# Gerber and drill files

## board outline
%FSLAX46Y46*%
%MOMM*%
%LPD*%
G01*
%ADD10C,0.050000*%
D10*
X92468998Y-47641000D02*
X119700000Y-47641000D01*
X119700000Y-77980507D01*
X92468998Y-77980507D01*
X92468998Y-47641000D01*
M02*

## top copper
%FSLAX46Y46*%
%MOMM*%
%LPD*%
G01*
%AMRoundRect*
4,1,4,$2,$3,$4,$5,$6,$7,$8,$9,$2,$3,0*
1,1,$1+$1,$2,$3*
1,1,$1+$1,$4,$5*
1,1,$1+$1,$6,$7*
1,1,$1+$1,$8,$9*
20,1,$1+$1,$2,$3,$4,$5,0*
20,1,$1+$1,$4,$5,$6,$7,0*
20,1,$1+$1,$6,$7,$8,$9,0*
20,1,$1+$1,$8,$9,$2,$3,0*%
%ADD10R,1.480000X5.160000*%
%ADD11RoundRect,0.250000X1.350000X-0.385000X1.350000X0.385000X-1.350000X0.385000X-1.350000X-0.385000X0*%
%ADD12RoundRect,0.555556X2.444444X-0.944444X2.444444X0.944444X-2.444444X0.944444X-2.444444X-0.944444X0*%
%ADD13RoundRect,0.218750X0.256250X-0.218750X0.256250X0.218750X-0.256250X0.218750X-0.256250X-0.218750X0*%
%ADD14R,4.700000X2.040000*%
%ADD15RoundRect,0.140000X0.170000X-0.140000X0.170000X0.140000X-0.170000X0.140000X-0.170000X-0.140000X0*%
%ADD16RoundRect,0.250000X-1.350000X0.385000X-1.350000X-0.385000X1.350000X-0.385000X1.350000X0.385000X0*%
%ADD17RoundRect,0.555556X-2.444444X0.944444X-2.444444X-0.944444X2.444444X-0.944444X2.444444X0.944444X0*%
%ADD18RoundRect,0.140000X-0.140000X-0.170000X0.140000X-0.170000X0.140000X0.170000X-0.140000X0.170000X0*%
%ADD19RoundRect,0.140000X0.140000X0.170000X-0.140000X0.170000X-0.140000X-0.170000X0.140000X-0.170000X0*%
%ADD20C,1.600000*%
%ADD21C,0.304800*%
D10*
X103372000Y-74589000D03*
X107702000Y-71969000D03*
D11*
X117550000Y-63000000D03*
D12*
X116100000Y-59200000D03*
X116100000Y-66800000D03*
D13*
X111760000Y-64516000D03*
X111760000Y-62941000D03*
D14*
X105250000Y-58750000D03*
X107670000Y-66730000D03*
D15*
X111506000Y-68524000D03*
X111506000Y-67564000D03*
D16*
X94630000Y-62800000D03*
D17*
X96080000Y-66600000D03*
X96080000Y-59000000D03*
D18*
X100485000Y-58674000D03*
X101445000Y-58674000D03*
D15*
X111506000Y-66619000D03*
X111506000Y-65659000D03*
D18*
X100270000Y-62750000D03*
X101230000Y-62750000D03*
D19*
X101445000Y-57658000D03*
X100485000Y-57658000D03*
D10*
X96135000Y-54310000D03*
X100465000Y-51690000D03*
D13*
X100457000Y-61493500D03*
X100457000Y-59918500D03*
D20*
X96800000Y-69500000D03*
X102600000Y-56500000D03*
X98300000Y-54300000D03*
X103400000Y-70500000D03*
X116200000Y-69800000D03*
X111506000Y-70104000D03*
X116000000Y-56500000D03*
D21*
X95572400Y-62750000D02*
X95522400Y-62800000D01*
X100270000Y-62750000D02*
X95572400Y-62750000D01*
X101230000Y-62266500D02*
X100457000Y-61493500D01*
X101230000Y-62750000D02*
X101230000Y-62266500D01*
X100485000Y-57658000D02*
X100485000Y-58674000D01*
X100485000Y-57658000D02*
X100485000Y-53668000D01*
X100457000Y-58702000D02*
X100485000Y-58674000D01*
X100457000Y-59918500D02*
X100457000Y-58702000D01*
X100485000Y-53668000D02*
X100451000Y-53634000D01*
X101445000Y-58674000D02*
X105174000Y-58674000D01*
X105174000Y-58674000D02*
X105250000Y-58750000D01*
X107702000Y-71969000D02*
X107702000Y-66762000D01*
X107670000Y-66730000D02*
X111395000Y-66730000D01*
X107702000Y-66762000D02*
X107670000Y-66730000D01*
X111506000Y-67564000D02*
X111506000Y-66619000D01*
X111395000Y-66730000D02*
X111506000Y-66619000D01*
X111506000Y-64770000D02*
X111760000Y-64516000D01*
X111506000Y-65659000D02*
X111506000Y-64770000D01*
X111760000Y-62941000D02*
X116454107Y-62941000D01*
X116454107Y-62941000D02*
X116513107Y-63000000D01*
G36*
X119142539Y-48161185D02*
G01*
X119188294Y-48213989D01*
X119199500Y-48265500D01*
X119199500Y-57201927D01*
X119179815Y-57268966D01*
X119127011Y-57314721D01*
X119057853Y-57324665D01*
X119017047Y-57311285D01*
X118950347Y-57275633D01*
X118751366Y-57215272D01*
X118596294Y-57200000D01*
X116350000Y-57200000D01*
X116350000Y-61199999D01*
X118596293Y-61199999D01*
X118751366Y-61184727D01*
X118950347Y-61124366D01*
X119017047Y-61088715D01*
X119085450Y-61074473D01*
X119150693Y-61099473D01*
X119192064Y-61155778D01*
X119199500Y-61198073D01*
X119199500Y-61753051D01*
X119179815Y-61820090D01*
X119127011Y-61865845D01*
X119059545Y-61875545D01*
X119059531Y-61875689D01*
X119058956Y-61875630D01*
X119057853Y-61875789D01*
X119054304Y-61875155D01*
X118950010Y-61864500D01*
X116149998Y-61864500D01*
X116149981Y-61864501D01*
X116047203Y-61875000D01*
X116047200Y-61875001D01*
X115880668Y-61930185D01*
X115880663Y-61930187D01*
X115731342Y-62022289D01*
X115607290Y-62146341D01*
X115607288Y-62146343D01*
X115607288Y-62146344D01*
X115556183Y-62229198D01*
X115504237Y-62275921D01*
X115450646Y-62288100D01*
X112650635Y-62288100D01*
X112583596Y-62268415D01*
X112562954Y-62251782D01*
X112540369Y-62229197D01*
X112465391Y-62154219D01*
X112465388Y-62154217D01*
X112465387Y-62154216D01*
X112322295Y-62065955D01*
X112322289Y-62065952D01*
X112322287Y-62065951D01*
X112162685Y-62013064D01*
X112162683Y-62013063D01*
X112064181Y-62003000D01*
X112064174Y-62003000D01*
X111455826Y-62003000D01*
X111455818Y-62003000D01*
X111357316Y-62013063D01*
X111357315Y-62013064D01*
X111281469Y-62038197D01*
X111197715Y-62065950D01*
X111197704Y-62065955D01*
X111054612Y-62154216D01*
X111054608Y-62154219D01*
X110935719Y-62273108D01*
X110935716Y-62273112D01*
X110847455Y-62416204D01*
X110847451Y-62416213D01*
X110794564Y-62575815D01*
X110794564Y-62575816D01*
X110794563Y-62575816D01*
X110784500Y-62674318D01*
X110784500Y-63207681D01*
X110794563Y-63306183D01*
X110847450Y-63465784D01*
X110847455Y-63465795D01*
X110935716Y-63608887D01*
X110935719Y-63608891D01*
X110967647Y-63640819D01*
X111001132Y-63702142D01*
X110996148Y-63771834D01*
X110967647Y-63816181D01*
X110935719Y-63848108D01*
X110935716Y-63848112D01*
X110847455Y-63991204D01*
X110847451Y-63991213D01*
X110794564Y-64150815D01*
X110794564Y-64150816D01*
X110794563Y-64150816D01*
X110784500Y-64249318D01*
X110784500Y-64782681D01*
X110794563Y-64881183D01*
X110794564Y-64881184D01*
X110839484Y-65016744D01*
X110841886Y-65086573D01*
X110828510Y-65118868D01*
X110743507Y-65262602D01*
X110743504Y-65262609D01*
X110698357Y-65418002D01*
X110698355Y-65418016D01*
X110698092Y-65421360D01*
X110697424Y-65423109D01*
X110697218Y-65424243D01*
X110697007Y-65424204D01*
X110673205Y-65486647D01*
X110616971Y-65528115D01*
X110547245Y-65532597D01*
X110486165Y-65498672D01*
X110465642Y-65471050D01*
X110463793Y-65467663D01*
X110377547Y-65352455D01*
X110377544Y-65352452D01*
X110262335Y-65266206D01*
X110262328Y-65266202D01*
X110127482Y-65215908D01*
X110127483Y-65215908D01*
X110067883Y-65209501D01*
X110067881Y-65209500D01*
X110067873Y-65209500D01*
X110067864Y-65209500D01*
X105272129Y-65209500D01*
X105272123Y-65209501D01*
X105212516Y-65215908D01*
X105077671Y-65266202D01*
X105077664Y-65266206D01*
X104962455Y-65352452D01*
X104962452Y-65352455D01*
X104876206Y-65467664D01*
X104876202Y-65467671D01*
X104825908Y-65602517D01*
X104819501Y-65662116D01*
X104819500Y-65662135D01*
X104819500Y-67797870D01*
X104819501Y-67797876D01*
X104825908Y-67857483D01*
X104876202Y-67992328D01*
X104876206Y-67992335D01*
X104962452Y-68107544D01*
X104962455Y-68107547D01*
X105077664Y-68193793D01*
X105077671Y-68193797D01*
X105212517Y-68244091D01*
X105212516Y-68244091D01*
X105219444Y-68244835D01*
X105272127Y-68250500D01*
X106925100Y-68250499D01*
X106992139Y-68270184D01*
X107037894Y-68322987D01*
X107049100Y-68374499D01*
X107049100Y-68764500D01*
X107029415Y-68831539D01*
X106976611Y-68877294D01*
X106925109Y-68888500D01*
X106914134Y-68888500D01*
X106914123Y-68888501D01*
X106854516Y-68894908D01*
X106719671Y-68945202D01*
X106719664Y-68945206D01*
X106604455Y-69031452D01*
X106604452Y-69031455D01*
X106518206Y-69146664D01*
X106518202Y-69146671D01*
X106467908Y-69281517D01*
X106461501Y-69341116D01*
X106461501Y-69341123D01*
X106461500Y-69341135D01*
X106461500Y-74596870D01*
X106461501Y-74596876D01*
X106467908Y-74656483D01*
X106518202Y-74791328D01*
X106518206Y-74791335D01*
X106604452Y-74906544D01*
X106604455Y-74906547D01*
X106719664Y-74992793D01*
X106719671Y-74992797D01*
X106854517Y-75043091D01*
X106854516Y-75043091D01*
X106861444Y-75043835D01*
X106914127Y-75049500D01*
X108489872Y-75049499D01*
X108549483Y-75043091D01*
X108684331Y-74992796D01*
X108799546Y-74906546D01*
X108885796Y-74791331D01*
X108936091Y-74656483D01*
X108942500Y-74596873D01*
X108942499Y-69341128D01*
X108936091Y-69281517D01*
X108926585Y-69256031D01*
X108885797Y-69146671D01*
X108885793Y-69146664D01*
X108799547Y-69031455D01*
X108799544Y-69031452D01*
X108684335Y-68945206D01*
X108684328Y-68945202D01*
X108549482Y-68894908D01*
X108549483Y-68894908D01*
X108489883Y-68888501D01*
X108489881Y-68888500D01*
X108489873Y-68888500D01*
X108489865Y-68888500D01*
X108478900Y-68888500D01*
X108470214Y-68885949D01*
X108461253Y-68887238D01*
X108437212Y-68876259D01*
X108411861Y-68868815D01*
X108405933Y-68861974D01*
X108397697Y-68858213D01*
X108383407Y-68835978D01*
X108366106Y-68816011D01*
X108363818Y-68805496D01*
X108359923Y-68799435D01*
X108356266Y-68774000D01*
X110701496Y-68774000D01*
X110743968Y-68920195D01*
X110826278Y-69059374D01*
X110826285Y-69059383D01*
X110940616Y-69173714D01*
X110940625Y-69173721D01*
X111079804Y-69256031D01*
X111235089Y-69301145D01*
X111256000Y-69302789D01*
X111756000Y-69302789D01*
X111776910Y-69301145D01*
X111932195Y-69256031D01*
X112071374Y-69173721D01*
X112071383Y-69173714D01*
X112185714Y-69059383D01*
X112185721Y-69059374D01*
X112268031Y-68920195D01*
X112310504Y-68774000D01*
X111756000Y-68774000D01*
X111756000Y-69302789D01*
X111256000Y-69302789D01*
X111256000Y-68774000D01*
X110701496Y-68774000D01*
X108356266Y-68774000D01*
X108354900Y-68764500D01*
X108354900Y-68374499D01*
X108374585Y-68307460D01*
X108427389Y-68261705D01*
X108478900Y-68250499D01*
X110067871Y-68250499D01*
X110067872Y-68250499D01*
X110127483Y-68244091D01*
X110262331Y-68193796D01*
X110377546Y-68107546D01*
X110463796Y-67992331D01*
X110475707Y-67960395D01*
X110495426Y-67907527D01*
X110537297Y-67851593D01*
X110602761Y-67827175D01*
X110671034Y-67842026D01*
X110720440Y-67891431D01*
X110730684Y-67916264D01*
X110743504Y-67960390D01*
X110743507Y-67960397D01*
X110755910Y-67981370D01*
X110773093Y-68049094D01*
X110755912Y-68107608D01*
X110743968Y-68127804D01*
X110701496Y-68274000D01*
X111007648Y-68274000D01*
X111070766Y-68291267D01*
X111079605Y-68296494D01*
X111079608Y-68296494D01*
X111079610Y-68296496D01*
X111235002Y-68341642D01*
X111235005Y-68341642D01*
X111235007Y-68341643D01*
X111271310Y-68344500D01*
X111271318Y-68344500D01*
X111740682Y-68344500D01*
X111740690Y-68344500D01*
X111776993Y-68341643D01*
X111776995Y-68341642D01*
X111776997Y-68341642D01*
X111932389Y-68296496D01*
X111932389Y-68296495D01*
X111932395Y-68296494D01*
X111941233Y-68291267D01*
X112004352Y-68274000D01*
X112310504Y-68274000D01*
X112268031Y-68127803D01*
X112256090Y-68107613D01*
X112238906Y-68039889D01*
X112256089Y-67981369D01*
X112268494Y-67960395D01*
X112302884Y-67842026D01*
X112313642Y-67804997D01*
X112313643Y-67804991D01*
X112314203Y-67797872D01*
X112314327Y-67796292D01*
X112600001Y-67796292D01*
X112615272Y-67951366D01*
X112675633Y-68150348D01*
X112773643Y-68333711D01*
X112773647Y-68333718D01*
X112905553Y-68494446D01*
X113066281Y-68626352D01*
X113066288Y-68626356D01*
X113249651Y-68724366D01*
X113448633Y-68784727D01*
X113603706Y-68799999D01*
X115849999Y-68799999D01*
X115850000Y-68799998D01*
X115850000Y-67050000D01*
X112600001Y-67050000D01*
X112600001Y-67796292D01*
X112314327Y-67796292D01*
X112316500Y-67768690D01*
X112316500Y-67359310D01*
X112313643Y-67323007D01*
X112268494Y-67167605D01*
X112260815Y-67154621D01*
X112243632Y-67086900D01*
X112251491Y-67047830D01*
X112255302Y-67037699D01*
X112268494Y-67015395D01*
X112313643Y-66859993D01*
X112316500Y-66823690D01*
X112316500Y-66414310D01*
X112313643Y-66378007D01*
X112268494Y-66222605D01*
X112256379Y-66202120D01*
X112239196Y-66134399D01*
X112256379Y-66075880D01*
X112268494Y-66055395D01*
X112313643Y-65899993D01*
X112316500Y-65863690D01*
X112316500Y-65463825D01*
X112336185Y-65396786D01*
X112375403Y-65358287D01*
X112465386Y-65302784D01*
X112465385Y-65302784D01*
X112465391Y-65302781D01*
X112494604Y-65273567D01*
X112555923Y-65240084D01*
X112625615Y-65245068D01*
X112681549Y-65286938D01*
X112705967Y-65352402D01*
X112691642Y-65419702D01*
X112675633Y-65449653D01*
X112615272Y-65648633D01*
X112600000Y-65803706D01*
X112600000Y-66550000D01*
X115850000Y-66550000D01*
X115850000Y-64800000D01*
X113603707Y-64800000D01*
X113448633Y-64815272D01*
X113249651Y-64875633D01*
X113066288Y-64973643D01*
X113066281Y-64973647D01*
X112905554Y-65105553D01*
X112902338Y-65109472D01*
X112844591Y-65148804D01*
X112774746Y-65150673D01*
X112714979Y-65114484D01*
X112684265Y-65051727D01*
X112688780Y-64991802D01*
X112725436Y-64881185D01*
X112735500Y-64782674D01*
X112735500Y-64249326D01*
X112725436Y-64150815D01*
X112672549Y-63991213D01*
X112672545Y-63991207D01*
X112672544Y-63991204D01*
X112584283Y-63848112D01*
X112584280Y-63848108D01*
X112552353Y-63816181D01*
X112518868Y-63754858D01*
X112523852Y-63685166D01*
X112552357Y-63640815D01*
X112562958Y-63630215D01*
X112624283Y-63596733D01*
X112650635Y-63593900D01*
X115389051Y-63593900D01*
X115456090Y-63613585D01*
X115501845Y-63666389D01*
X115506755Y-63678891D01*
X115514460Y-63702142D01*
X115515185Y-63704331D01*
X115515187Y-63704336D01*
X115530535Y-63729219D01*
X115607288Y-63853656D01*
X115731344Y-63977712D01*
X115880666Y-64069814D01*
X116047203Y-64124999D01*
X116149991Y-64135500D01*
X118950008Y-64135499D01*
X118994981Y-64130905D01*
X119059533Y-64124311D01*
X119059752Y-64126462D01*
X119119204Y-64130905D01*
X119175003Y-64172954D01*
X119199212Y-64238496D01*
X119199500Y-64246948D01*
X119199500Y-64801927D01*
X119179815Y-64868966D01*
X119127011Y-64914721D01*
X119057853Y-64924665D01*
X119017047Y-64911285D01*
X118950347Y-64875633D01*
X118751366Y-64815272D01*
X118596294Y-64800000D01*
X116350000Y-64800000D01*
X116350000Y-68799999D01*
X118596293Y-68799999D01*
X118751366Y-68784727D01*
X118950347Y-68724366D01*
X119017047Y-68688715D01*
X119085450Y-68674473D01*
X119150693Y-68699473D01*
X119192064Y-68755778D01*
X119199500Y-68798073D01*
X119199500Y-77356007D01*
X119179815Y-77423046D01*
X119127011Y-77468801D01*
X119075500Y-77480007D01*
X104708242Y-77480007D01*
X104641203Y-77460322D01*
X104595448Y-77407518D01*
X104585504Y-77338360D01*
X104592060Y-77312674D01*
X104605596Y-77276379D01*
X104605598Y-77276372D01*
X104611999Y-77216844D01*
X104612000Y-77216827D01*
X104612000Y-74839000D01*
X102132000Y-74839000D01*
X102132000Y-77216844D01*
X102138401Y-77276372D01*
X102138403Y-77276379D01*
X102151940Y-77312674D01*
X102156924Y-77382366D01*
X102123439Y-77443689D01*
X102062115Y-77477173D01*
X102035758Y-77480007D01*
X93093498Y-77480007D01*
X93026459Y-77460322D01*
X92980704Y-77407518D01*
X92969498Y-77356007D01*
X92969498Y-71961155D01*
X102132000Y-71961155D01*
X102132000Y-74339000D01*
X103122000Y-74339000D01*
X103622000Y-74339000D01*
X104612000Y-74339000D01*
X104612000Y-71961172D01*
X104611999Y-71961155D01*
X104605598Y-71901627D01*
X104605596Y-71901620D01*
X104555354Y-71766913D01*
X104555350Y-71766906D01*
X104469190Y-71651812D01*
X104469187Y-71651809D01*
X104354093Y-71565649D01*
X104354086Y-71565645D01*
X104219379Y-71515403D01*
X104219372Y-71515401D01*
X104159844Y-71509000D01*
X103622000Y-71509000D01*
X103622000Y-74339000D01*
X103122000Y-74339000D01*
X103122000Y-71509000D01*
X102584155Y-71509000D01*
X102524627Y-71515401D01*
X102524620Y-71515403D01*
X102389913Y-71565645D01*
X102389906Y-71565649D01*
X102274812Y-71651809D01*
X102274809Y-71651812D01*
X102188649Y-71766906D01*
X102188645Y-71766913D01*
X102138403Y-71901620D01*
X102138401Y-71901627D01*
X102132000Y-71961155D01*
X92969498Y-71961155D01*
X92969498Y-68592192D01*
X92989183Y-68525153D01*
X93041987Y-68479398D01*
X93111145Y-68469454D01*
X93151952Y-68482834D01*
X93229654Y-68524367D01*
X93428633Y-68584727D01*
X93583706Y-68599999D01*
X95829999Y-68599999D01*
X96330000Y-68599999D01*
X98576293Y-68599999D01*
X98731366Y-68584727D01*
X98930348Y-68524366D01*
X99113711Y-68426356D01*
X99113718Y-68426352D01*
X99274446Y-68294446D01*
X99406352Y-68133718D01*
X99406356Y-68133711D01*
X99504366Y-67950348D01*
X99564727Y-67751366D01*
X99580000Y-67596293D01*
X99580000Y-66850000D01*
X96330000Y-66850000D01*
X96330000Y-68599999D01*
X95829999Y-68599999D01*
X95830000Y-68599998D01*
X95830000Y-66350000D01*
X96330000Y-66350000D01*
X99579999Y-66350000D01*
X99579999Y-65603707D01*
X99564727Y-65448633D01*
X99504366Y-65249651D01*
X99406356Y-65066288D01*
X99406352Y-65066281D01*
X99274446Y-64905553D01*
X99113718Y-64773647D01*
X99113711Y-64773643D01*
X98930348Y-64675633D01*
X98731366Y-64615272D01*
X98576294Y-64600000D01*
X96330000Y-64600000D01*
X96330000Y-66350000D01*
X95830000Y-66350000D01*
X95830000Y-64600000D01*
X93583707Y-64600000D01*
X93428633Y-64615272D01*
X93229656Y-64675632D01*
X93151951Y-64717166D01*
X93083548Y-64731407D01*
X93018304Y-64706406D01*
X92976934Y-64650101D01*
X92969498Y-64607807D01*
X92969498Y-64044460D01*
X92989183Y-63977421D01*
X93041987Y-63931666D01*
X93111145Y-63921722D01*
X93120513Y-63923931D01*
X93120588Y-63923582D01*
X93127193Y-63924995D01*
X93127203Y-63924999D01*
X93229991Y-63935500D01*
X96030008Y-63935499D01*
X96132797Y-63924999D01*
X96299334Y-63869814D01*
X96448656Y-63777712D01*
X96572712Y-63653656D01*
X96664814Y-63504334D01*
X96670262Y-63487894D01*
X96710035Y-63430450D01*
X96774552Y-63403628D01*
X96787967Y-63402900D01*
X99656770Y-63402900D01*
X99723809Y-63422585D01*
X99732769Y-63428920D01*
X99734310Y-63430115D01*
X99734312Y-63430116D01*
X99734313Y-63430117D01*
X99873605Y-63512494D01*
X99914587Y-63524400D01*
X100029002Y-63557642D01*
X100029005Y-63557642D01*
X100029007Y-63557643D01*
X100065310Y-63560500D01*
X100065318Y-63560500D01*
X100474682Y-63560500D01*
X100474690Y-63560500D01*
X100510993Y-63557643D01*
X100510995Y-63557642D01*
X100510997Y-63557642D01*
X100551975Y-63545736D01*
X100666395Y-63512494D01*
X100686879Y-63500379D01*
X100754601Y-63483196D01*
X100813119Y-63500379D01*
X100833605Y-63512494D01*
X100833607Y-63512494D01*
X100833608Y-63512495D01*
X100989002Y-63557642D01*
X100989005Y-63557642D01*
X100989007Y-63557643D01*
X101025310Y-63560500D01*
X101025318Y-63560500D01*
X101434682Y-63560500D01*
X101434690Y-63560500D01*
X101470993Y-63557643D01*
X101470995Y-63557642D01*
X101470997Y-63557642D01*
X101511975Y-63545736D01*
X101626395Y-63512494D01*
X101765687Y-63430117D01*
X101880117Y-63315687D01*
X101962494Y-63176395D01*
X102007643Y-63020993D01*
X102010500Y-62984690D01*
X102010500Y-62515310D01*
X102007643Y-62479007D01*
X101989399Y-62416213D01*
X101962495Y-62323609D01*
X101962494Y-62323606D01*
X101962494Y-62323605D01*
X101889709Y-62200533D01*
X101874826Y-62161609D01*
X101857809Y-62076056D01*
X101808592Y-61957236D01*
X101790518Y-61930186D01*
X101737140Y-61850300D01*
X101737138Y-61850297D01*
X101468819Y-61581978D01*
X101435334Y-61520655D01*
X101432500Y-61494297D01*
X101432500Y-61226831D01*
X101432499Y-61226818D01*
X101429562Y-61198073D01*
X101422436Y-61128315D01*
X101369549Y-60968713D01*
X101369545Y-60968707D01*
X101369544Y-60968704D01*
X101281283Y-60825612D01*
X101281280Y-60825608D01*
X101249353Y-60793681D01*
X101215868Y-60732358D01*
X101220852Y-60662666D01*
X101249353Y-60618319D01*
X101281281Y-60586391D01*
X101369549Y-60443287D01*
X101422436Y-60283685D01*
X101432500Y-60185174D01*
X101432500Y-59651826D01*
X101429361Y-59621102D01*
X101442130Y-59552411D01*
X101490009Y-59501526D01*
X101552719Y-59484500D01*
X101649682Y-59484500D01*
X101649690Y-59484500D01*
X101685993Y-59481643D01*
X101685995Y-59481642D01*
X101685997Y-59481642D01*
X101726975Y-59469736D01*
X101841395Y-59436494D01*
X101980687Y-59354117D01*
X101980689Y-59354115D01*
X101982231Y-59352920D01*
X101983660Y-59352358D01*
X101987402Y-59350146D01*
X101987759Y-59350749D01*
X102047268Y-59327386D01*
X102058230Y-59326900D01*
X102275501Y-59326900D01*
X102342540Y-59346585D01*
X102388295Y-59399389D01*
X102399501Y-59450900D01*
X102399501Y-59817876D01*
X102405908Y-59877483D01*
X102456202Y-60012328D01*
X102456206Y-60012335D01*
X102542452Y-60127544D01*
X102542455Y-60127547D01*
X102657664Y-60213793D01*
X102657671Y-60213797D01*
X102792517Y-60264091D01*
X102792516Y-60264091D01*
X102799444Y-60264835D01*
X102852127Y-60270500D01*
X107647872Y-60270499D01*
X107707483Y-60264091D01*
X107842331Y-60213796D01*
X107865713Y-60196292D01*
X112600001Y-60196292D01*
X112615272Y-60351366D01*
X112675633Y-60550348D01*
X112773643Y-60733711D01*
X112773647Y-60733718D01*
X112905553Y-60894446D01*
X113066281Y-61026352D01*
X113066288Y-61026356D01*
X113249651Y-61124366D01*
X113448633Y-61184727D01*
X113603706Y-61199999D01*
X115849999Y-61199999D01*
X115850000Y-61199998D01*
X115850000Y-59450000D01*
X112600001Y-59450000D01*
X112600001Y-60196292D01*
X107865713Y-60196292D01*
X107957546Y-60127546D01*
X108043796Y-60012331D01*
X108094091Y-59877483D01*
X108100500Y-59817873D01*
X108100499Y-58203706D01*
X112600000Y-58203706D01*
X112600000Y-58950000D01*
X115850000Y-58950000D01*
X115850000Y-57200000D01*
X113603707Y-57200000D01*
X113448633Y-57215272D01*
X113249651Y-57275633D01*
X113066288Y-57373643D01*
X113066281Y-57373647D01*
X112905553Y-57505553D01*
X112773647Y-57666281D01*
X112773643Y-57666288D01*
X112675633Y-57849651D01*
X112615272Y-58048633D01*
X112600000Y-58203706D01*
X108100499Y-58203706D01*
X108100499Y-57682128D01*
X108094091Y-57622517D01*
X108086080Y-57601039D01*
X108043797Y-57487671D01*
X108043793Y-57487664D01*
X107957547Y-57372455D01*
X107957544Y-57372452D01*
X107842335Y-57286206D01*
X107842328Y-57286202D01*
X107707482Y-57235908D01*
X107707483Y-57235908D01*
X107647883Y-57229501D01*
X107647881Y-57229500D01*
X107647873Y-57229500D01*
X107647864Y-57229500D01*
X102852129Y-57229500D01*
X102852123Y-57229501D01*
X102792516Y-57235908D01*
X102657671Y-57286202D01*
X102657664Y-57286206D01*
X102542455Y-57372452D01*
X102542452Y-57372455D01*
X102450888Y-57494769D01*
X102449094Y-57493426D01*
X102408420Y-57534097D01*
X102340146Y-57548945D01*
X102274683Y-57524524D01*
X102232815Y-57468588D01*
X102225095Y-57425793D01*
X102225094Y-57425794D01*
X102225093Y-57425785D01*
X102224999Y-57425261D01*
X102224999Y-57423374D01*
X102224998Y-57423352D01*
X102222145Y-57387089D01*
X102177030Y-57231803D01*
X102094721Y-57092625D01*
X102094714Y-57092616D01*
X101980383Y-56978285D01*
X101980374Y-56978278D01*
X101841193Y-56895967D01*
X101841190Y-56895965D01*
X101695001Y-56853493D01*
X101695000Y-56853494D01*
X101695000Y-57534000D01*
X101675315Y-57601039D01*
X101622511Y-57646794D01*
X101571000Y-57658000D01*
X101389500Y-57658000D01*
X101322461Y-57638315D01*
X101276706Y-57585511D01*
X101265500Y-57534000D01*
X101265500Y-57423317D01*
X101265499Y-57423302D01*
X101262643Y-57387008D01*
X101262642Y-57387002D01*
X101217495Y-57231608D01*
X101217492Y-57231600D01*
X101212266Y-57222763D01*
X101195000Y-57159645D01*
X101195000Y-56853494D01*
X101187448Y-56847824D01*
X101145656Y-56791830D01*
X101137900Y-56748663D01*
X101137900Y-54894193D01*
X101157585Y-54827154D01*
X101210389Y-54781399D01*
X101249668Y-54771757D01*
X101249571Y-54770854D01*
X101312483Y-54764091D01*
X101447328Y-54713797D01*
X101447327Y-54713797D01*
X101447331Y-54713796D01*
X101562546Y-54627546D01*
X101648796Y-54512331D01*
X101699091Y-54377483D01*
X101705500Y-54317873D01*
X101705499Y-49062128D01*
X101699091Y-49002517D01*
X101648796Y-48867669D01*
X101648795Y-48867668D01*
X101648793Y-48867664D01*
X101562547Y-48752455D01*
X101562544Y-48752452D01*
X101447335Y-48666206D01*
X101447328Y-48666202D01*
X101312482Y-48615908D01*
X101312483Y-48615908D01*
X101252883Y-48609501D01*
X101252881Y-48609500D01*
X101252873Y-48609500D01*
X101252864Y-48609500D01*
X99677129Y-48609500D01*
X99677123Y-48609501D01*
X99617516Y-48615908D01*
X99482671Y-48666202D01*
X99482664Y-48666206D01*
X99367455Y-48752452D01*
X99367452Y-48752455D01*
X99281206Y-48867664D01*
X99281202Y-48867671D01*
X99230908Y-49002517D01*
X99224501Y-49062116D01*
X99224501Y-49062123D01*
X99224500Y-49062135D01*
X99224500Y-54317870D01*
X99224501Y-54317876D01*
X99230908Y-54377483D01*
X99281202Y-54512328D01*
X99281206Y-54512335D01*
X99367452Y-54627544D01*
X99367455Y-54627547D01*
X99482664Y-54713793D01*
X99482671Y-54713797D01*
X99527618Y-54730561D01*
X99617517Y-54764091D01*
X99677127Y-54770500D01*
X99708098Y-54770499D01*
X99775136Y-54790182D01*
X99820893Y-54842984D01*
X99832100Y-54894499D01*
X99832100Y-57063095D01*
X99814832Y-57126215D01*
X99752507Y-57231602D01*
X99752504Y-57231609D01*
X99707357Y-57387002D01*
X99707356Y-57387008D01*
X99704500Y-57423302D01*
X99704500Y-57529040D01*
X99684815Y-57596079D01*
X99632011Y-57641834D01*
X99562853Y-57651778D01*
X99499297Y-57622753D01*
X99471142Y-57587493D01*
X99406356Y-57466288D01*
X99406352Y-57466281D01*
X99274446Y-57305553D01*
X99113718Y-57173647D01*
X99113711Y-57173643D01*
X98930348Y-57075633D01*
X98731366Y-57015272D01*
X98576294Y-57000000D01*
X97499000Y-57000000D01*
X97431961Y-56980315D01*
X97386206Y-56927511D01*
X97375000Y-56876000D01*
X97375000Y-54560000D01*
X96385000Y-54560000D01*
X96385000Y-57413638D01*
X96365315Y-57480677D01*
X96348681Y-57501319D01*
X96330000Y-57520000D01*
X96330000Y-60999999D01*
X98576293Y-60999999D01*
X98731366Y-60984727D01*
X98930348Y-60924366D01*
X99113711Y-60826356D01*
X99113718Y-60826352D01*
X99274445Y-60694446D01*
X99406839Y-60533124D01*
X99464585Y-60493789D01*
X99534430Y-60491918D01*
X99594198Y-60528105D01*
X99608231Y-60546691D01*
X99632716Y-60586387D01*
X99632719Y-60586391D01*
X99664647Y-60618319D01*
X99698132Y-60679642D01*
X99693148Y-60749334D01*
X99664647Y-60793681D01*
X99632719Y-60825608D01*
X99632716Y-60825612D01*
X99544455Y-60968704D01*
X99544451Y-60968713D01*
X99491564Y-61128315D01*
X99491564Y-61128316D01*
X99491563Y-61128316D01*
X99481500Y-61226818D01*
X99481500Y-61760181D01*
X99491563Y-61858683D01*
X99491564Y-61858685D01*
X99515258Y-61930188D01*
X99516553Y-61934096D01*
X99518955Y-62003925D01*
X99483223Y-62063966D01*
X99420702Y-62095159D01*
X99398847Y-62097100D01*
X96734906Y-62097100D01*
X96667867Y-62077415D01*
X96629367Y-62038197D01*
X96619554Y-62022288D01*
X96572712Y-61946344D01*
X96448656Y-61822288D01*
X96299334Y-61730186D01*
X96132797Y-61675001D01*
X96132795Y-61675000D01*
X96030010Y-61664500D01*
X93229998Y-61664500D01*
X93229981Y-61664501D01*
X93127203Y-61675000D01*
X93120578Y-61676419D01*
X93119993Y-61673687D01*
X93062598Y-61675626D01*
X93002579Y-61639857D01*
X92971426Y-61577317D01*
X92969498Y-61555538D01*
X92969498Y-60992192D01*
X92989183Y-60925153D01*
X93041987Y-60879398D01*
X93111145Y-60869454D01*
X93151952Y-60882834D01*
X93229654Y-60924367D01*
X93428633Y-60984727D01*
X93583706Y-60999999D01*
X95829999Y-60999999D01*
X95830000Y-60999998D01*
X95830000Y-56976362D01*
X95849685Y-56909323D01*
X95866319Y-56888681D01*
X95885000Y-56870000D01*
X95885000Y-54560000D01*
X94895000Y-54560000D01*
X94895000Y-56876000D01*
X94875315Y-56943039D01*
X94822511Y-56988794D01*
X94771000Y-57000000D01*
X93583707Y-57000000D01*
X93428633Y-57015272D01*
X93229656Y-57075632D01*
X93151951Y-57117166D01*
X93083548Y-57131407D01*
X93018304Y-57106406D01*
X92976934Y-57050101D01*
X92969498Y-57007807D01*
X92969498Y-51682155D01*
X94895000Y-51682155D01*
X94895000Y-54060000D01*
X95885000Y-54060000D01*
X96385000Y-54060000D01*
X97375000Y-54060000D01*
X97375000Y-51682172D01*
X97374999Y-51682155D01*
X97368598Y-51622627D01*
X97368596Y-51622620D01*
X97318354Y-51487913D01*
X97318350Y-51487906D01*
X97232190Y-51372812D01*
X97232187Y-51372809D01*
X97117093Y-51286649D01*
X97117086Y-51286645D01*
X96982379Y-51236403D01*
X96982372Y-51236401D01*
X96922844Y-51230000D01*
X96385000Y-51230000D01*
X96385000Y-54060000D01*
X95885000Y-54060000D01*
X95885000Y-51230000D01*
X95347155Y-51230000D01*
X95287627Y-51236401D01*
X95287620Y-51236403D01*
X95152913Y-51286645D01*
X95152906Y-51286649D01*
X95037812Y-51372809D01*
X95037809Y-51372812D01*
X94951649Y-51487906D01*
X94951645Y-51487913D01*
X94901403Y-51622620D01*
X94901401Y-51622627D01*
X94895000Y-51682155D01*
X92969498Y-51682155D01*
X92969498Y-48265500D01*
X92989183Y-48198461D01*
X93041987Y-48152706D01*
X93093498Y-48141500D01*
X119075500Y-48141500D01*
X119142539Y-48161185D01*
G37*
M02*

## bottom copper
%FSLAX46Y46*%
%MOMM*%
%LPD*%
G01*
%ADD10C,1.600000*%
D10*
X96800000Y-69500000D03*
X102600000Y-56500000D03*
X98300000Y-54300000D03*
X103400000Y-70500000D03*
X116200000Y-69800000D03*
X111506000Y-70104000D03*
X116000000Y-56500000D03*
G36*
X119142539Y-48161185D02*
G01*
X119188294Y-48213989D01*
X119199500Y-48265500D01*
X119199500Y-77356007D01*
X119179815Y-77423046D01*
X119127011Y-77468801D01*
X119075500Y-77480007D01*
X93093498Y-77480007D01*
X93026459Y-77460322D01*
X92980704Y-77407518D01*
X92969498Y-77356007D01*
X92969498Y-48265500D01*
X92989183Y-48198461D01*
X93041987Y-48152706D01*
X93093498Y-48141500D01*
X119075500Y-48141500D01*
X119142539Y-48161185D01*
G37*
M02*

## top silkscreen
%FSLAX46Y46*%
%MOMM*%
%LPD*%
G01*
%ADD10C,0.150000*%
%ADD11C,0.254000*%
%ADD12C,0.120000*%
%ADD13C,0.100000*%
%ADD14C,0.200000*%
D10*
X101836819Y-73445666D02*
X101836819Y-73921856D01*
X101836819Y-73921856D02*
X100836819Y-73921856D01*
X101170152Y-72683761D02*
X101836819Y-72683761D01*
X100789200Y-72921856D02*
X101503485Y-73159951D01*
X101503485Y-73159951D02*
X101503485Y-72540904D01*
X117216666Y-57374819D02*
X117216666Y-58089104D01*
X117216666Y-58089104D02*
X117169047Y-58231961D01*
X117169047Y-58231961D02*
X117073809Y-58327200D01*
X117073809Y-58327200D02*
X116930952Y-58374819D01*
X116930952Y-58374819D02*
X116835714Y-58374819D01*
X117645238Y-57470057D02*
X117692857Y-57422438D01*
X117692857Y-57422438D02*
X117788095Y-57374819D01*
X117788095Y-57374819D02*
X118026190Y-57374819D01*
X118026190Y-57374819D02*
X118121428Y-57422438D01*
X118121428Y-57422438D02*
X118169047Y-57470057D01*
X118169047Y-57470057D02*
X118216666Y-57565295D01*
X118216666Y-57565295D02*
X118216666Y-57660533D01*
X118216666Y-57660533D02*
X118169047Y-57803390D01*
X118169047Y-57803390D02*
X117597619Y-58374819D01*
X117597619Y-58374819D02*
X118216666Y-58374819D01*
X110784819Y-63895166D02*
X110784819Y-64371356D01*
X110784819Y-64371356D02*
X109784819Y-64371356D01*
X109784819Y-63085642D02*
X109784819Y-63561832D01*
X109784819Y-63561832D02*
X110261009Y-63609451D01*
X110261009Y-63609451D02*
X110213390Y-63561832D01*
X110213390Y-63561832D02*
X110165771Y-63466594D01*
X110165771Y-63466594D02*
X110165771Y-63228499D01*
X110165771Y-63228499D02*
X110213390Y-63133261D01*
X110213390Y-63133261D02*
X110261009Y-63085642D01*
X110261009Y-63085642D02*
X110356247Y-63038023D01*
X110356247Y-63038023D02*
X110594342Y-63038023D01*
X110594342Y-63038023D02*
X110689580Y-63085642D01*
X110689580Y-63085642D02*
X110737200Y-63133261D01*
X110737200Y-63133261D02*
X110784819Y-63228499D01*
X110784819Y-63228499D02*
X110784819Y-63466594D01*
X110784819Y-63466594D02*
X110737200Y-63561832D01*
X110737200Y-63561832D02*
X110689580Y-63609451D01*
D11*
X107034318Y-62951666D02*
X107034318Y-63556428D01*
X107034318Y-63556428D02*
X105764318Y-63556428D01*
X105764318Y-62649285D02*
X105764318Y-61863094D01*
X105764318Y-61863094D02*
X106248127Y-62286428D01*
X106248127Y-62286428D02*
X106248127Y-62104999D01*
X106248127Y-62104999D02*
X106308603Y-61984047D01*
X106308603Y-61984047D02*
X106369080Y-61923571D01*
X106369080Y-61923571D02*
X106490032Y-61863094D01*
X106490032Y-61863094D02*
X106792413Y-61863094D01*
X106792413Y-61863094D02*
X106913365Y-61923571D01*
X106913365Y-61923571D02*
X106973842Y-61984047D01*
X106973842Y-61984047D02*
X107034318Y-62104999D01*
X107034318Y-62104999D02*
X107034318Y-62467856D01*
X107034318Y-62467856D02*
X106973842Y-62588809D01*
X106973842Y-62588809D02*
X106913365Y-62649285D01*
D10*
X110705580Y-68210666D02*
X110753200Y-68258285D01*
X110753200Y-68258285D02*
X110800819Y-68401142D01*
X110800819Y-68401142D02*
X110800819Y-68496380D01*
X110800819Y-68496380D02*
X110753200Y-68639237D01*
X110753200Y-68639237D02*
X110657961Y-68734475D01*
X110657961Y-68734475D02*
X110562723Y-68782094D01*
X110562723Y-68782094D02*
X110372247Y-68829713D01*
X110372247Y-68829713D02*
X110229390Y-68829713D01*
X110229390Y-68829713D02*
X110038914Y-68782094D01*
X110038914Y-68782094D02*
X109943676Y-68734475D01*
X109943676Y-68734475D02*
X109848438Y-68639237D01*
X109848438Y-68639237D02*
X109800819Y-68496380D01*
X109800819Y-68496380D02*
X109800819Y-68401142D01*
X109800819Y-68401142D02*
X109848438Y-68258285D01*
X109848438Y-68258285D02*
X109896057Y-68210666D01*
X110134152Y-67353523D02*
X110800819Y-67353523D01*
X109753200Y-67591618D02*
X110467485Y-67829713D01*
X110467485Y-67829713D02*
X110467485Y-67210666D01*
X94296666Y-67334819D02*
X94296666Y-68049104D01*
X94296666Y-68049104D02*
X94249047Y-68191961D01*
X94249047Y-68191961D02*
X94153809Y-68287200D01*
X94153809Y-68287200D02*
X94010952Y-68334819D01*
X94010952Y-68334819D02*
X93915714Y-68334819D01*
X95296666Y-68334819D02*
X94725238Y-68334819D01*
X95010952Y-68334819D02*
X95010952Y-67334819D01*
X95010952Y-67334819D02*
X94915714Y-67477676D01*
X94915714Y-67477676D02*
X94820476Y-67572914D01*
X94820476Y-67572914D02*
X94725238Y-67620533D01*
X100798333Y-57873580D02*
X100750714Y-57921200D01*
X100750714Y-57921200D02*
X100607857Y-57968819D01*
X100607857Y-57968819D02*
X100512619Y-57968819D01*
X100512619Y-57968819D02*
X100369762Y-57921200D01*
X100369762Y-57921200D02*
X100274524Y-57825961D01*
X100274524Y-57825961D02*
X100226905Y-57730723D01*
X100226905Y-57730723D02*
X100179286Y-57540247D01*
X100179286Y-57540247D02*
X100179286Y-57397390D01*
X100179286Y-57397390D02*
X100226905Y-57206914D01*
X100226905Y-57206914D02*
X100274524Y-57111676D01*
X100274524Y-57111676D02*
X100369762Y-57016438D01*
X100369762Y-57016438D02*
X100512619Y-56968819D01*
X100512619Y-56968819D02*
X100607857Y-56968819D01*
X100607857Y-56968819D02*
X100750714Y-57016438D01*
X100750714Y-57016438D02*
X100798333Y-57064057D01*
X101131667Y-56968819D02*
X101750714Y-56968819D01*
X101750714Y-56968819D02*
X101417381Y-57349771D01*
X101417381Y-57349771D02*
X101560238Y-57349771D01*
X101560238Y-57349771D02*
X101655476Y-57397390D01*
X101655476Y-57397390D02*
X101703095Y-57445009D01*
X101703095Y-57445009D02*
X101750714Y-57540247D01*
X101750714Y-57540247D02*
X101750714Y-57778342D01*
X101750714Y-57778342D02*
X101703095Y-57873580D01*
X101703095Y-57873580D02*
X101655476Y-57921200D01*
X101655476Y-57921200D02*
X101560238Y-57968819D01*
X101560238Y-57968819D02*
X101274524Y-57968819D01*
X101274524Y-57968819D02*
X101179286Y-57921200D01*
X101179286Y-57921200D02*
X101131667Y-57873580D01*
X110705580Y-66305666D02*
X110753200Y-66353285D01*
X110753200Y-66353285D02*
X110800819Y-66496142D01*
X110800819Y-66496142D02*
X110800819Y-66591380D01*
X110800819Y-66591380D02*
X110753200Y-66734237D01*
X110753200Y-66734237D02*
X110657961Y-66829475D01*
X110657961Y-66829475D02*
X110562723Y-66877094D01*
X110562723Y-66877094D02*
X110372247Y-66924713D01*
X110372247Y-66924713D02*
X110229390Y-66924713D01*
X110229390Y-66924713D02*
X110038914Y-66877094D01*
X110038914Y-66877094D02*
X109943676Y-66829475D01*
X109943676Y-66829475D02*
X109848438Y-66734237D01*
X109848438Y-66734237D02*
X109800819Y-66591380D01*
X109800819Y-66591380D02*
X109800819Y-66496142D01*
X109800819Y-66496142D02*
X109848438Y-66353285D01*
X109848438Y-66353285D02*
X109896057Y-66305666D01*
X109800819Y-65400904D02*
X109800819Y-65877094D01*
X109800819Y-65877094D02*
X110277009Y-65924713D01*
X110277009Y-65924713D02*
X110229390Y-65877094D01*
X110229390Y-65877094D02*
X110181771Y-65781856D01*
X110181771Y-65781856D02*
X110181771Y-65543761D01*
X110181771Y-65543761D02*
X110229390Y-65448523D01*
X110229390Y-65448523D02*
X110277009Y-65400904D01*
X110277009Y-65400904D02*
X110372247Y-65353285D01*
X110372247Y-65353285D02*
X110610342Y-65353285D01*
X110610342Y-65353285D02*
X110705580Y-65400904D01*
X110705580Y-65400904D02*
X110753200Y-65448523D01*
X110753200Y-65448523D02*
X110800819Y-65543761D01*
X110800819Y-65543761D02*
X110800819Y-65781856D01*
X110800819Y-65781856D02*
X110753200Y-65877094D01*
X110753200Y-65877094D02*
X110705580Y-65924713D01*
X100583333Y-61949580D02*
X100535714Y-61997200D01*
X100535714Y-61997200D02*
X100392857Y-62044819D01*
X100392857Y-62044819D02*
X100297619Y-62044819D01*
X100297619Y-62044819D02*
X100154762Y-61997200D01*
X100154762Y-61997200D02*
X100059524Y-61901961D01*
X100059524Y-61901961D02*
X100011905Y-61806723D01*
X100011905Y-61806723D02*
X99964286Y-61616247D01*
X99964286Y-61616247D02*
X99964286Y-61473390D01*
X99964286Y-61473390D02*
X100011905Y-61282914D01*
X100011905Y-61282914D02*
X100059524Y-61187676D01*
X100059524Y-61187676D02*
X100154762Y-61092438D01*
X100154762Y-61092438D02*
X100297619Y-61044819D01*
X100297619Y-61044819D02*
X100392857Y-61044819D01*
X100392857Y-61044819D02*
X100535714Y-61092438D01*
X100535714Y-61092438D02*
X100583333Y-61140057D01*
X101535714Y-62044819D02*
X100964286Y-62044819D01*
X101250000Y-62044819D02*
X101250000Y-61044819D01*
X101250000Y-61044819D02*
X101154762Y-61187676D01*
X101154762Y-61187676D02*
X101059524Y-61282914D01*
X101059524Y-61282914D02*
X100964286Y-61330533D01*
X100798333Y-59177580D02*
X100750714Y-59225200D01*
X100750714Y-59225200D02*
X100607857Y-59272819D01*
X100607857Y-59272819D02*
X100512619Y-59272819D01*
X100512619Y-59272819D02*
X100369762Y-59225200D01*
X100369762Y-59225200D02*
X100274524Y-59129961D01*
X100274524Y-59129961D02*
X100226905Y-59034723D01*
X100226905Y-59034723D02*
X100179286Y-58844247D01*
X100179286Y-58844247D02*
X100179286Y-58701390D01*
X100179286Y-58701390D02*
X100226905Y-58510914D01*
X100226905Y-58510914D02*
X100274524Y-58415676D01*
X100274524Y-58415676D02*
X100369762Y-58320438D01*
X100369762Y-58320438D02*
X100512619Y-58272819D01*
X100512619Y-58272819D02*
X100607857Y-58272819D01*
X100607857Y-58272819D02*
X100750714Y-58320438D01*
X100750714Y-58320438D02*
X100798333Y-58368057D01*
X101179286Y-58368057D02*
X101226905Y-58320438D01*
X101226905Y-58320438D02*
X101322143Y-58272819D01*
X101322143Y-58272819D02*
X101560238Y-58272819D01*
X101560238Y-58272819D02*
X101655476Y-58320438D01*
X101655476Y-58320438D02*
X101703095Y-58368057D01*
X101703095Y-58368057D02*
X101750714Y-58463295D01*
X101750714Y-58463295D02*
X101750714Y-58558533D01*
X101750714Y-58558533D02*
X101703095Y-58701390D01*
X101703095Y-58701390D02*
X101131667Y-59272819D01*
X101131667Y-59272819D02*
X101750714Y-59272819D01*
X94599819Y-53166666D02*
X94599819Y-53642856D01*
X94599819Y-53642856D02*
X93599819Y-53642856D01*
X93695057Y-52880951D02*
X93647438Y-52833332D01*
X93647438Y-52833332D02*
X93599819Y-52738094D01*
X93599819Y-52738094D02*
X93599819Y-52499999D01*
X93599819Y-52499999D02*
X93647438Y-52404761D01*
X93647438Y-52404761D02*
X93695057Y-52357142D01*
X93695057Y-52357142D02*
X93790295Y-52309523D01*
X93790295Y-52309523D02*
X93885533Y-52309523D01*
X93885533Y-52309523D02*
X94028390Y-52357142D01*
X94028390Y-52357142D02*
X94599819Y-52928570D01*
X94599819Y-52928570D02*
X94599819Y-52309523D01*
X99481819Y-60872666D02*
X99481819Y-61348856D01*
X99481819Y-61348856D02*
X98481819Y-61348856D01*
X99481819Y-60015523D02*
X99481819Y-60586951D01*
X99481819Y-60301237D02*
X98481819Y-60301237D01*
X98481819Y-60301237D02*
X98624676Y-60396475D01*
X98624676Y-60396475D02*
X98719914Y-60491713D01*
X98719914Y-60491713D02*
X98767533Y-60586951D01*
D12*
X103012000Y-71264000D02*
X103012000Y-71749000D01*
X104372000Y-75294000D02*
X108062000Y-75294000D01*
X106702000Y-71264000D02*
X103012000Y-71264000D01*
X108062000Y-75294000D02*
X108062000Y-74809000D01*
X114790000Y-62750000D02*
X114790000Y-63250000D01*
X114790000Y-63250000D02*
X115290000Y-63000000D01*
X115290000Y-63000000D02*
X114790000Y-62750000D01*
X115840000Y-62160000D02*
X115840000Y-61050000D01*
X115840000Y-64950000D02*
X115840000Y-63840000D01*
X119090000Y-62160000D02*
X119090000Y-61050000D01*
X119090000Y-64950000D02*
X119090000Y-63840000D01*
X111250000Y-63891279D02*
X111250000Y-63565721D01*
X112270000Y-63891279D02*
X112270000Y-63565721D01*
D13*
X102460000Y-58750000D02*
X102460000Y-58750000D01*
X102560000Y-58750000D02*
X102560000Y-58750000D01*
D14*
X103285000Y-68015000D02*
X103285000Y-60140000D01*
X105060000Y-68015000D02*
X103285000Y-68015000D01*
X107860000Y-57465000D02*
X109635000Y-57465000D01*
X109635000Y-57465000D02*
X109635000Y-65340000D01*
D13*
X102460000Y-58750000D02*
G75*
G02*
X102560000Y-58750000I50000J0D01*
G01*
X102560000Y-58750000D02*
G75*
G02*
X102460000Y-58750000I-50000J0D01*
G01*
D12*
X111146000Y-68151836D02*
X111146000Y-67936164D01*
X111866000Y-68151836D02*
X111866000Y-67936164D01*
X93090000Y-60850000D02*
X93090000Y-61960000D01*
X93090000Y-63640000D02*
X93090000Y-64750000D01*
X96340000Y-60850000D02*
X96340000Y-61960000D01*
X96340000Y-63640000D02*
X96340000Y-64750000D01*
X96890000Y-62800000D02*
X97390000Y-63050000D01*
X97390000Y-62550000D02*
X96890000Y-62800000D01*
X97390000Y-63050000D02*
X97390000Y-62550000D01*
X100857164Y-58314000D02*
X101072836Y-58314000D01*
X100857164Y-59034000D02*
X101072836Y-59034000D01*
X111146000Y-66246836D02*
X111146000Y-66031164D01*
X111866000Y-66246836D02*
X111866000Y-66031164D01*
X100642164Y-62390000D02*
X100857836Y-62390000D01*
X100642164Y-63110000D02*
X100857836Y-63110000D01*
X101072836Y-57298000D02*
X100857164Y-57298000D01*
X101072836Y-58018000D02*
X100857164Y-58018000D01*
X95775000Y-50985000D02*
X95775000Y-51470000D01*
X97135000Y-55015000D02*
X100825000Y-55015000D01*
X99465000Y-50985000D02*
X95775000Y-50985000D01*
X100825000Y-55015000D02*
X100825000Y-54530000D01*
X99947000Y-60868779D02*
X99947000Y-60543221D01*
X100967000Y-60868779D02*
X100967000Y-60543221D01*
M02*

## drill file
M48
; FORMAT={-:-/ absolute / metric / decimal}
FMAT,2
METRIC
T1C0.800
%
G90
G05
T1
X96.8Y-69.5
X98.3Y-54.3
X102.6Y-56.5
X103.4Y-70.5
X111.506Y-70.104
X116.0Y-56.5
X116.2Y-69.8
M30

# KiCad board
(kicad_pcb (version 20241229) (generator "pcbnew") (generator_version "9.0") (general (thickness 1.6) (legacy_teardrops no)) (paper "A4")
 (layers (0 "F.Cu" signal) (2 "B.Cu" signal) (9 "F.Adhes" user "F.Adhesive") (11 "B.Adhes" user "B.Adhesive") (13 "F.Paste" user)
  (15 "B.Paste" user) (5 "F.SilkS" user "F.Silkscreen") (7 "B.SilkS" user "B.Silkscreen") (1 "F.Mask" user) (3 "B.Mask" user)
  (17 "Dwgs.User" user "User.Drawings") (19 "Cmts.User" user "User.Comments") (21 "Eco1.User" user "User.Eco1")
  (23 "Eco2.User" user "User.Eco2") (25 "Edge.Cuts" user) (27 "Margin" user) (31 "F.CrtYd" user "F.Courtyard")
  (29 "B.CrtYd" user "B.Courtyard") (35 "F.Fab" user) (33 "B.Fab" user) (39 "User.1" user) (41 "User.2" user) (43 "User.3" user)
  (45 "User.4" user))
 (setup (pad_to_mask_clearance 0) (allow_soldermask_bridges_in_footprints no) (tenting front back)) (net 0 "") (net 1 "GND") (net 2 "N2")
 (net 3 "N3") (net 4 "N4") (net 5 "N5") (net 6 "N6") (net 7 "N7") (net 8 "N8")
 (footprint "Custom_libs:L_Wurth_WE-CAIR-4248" (layer "F.Cu") (at 105.537 73.279 90)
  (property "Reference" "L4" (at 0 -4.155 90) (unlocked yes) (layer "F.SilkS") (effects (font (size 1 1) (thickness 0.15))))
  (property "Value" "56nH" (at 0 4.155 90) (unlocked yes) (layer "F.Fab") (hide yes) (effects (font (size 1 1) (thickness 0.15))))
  (fp_line (start 2.015 -2.525) (end 1.53 -2.525) (stroke (width 0.12) (type solid)) (layer "F.SilkS"))
  (fp_line (start -2.015 -1.165) (end -2.015 2.525) (stroke (width 0.12) (type solid)) (layer "F.SilkS"))
  (fp_line (start 2.015 1.165) (end 2.015 -2.525) (stroke (width 0.12) (type solid)) (layer "F.SilkS"))
  (fp_line (start -2.015 2.525) (end -1.53 2.525) (stroke (width 0.12) (type solid)) (layer "F.SilkS"))
  (pad "1" smd rect (at -1.31 -2.165 90) (size 5.16 1.48) (layers "F.Cu" "F.Mask" "F.Paste") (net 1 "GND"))
  (pad "2" smd rect (at 1.31 2.165 90) (size 5.16 1.48) (layers "F.Cu" "F.Mask" "F.Paste") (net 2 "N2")))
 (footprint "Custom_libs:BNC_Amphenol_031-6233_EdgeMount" (layer "F.Cu") (at 117.55 63)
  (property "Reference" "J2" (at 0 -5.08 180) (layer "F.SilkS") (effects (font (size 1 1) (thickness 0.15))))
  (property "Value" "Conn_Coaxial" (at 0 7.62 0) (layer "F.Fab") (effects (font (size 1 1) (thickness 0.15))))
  (fp_line (start -2.76 -0.25) (end -2.76 0.25) (stroke (width 0.12) (type solid)) (layer "F.SilkS"))
  (fp_line (start -2.76 0.25) (end -2.26 0) (stroke (width 0.12) (type solid)) (layer "F.SilkS"))
  (fp_line (start -2.26 0) (end -2.76 -0.25) (stroke (width 0.12) (type solid)) (layer "F.SilkS"))
  (fp_line (start -1.71 -0.84) (end -1.71 -1.95) (stroke (width 0.12) (type solid)) (layer "F.SilkS"))
  (fp_line (start -1.71 1.95) (end -1.71 0.84) (stroke (width 0.12) (type solid)) (layer "F.SilkS"))
  (fp_line (start 1.54 -0.84) (end 1.54 -1.95) (stroke (width 0.12) (type solid)) (layer "F.SilkS"))
  (fp_line (start 1.54 1.95) (end 1.54 0.84) (stroke (width 0.12) (type solid)) (layer "F.SilkS"))
  (pad "1" smd roundrect (at 0 0 90) (size 1.27 3.2) (layers "F.Cu" "F.Mask") (roundrect_rratio 0.1968503937) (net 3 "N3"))
  (pad "2" smd roundrect (at -1.45 -3.8 90) (size 3 6) (layers "F.Cu" "F.Mask") (roundrect_rratio 0.1851851852) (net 1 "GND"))
  (pad "2" smd roundrect (at -1.45 3.8 90) (size 3 6) (layers "F.Cu" "F.Mask") (roundrect_rratio 0.1851851852) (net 1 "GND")))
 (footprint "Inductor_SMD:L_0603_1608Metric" (layer "F.Cu") (at 111.76 63.7285 90)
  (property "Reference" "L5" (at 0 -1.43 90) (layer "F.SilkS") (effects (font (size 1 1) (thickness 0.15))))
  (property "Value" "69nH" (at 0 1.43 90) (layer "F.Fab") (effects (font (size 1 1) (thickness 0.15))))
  (fp_line (start -0.162779 -0.51) (end 0.162779 -0.51) (stroke (width 0.12) (type solid)) (layer "F.SilkS"))
  (fp_line (start -0.162779 0.51) (end 0.162779 0.51) (stroke (width 0.12) (type solid)) (layer "F.SilkS"))
  (pad "1" smd roundrect (at -0.7875 0 90) (size 0.875 0.95) (layers "F.Cu" "F.Mask" "F.Paste") (roundrect_rratio 0.25) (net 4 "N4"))
  (pad "2" smd roundrect (at 0.7875 0 90) (size 0.875 0.95) (layers "F.Cu" "F.Mask" "F.Paste") (roundrect_rratio 0.25) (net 3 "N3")))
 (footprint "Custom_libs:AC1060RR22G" (layer "F.Cu") (at 106.46 62.74 -90)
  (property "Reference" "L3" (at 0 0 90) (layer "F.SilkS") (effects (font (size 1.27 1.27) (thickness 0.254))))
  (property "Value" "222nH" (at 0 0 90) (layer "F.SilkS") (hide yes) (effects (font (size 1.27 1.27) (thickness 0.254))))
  (fp_line (start -3.99 4) (end -3.99 4) (stroke (width 0.1) (type solid)) (layer "F.SilkS"))
  (fp_line (start -3.99 3.9) (end -3.99 3.9) (stroke (width 0.1) (type solid)) (layer "F.SilkS"))
  (fp_line (start 5.275 3.175) (end -2.6 3.175) (stroke (width 0.2) (type solid)) (layer "F.SilkS"))
  (fp_line (start 5.275 1.4) (end 5.275 3.175) (stroke (width 0.2) (type solid)) (layer "F.SilkS"))
  (fp_line (start -5.275 -1.4) (end -5.275 -3.175) (stroke (width 0.2) (type solid)) (layer "F.SilkS"))
  (fp_line (start -5.275 -3.175) (end 2.6 -3.175) (stroke (width 0.2) (type solid)) (layer "F.SilkS"))
  (fp_arc (start -3.99 4) (mid -4.04 3.95) (end -3.99 3.9) (stroke (width 0.1) (type solid)) (layer "F.SilkS"))
  (fp_arc (start -3.99 3.9) (mid -3.94 3.95) (end -3.99 4) (stroke (width 0.1) (type solid)) (layer "F.SilkS"))
  (pad "1" smd rect (at -3.99 1.21 270) (size 2.04 4.7) (layers "F.Cu" "F.Mask" "F.Paste") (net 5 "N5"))
  (pad "2" smd rect (at 3.99 -1.21 270) (size 2.04 4.7) (layers "F.Cu" "F.Mask" "F.Paste") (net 2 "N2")))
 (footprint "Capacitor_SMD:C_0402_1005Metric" (layer "F.Cu") (at 111.506 68.044 90)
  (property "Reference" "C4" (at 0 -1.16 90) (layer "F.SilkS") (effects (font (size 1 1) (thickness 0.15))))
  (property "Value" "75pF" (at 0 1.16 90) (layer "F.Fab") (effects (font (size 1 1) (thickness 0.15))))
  (fp_line (start -0.107836 -0.36) (end 0.107836 -0.36) (stroke (width 0.12) (type solid)) (layer "F.SilkS"))
  (fp_line (start -0.107836 0.36) (end 0.107836 0.36) (stroke (width 0.12) (type solid)) (layer "F.SilkS"))
  (pad "1" smd roundrect (at -0.48 0 90) (size 0.56 0.62) (layers "F.Cu" "F.Mask" "F.Paste") (roundrect_rratio 0.25) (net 1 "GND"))
  (pad "2" smd roundrect (at 0.48 0 90) (size 0.56 0.62) (layers "F.Cu" "F.Mask" "F.Paste") (roundrect_rratio 0.25) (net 2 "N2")))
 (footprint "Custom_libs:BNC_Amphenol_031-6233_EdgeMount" (layer "F.Cu") (at 94.63 62.8 180)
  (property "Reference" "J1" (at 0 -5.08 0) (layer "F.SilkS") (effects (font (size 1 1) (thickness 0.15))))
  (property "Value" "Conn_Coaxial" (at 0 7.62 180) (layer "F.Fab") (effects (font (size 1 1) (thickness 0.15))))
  (fp_line (start 1.54 1.95) (end 1.54 0.84) (stroke (width 0.12) (type solid)) (layer "F.SilkS"))
  (fp_line (start 1.54 -0.84) (end 1.54 -1.95) (stroke (width 0.12) (type solid)) (layer "F.SilkS"))
  (fp_line (start -1.71 1.95) (end -1.71 0.84) (stroke (width 0.12) (type solid)) (layer "F.SilkS"))
  (fp_line (start -1.71 -0.84) (end -1.71 -1.95) (stroke (width 0.12) (type solid)) (layer "F.SilkS"))
  (fp_line (start -2.26 0) (end -2.76 -0.25) (stroke (width 0.12) (type solid)) (layer "F.SilkS"))
  (fp_line (start -2.76 0.25) (end -2.26 0) (stroke (width 0.12) (type solid)) (layer "F.SilkS"))
  (fp_line (start -2.76 -0.25) (end -2.76 0.25) (stroke (width 0.12) (type solid)) (layer "F.SilkS"))
  (pad "1" smd roundrect (at 0 0 270) (size 1.27 3.2) (layers "F.Cu" "F.Mask") (roundrect_rratio 0.1968503937) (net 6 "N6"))
  (pad "2" smd roundrect (at -1.45 -3.8 270) (size 3 6) (layers "F.Cu" "F.Mask") (roundrect_rratio 0.1851851852) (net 1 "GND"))
  (pad "2" smd roundrect (at -1.45 3.8 270) (size 3 6) (layers "F.Cu" "F.Mask") (roundrect_rratio 0.1851851852) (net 1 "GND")))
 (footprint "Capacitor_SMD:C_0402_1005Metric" (layer "F.Cu") (at 100.965 58.674)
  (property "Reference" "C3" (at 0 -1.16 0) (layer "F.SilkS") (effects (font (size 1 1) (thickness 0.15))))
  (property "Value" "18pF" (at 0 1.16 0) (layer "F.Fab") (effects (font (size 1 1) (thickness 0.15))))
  (fp_line (start -0.107836 -0.36) (end 0.107836 -0.36) (stroke (width 0.12) (type solid)) (layer "F.SilkS"))
  (fp_line (start -0.107836 0.36) (end 0.107836 0.36) (stroke (width 0.12) (type solid)) (layer "F.SilkS"))
  (pad "1" smd roundrect (at -0.48 0) (size 0.56 0.62) (layers "F.Cu" "F.Mask" "F.Paste") (roundrect_rratio 0.25) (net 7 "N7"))
  (pad "2" smd roundrect (at 0.48 0) (size 0.56 0.62) (layers "F.Cu" "F.Mask" "F.Paste") (roundrect_rratio 0.25) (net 5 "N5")))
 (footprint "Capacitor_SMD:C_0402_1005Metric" (layer "F.Cu") (at 111.506 66.139 90)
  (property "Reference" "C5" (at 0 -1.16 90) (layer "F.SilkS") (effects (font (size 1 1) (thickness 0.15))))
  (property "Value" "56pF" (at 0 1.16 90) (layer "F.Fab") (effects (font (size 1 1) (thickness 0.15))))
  (fp_line (start -0.107836 -0.36) (end 0.107836 -0.36) (stroke (width 0.12) (type solid)) (layer "F.SilkS"))
  (fp_line (start -0.107836 0.36) (end 0.107836 0.36) (stroke (width 0.12) (type solid)) (layer "F.SilkS"))
  (pad "1" smd roundrect (at -0.48 0 90) (size 0.56 0.62) (layers "F.Cu" "F.Mask" "F.Paste") (roundrect_rratio 0.25) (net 2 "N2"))
  (pad "2" smd roundrect (at 0.48 0 90) (size 0.56 0.62) (layers "F.Cu" "F.Mask" "F.Paste") (roundrect_rratio 0.25) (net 4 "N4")))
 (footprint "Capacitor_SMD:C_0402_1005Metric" (layer "F.Cu") (at 100.75 62.75)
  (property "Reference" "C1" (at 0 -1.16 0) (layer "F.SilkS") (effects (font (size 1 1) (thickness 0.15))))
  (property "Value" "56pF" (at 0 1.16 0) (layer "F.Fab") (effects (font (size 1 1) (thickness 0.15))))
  (fp_line (start -0.107836 -0.36) (end 0.107836 -0.36) (stroke (width 0.12) (type solid)) (layer "F.SilkS"))
  (fp_line (start -0.107836 0.36) (end 0.107836 0.36) (stroke (width 0.12) (type solid)) (layer "F.SilkS"))
  (pad "1" smd roundrect (at -0.48 0) (size 0.56 0.62) (layers "F.Cu" "F.Mask" "F.Paste") (roundrect_rratio 0.25) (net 6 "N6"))
  (pad "2" smd roundrect (at 0.48 0) (size 0.56 0.62) (layers "F.Cu" "F.Mask" "F.Paste") (roundrect_rratio 0.25) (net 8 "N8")))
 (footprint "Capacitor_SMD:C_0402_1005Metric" (layer "F.Cu") (at 100.965 57.658 180)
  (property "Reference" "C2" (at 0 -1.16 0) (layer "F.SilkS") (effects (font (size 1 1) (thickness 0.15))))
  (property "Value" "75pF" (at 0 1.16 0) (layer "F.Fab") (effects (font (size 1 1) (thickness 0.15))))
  (fp_line (start -0.107836 0.36) (end 0.107836 0.36) (stroke (width 0.12) (type solid)) (layer "F.SilkS"))
  (fp_line (start -0.107836 -0.36) (end 0.107836 -0.36) (stroke (width 0.12) (type solid)) (layer "F.SilkS"))
  (pad "1" smd roundrect (at -0.48 0 180) (size 0.56 0.62) (layers "F.Cu" "F.Mask" "F.Paste") (roundrect_rratio 0.25) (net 1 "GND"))
  (pad "2" smd roundrect (at 0.48 0 180) (size 0.56 0.62) (layers "F.Cu" "F.Mask" "F.Paste") (roundrect_rratio 0.25) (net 7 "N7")))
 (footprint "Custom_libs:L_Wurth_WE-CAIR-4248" (layer "F.Cu") (at 98.3 53 90)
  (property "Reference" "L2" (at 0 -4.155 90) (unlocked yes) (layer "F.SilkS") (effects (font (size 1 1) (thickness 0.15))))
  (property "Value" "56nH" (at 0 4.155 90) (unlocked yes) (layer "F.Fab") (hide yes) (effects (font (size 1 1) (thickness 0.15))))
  (fp_line (start 2.015 -2.525) (end 1.53 -2.525) (stroke (width 0.12) (type solid)) (layer "F.SilkS"))
  (fp_line (start -2.015 -1.165) (end -2.015 2.525) (stroke (width 0.12) (type solid)) (layer "F.SilkS"))
  (fp_line (start 2.015 1.165) (end 2.015 -2.525) (stroke (width 0.12) (type solid)) (layer "F.SilkS"))
  (fp_line (start -2.015 2.525) (end -1.53 2.525) (stroke (width 0.12) (type solid)) (layer "F.SilkS"))
  (pad "1" smd rect (at -1.31 -2.165 90) (size 5.16 1.48) (layers "F.Cu" "F.Mask" "F.Paste") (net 1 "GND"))
  (pad "2" smd rect (at 1.31 2.165 90) (size 5.16 1.48) (layers "F.Cu" "F.Mask" "F.Paste") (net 7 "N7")))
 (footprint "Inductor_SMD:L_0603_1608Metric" (layer "F.Cu") (at 100.457 60.706 90)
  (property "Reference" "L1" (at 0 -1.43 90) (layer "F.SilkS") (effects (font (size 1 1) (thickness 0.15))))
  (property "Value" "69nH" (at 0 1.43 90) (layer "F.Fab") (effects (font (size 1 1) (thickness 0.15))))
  (fp_line (start -0.162779 -0.51) (end 0.162779 -0.51) (stroke (width 0.12) (type solid)) (layer "F.SilkS"))
  (fp_line (start -0.162779 0.51) (end 0.162779 0.51) (stroke (width 0.12) (type solid)) (layer "F.SilkS"))
  (pad "1" smd roundrect (at -0.7875 0 90) (size 0.875 0.95) (layers "F.Cu" "F.Mask" "F.Paste") (roundrect_rratio 0.25) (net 8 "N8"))
  (pad "2" smd roundrect (at 0.7875 0 90) (size 0.875 0.95) (layers "F.Cu" "F.Mask" "F.Paste") (roundrect_rratio 0.25) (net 7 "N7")))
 (gr_rect (start 92.468998 47.641) (end 119.7 77.980507) (stroke (width 0.05) (type default)) (fill no) (layer "Edge.Cuts"))
 (segment (start 95.5724 62.75) (end 95.5224 62.8) (width 0.3048) (layer "F.Cu") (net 6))
 (segment (start 100.27 62.75) (end 95.5724 62.75) (width 0.3048) (layer "F.Cu") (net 6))
 (segment (start 101.23 62.2665) (end 100.457 61.4935) (width 0.3048) (layer "F.Cu") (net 8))
 (segment (start 101.23 62.75) (end 101.23 62.2665) (width 0.3048) (layer "F.Cu") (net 8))
 (segment (start 100.485 57.658) (end 100.485 58.674) (width 0.3048) (layer "F.Cu") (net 7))
 (segment (start 100.485 57.658) (end 100.485 53.668) (width 0.3048) (layer "F.Cu") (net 7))
 (segment (start 100.457 58.702) (end 100.485 58.674) (width 0.3048) (layer "F.Cu") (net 7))
 (segment (start 100.457 59.9185) (end 100.457 58.702) (width 0.3048) (layer "F.Cu") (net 7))
 (segment (start 100.485 53.668) (end 100.451 53.634) (width 0.3048) (layer "F.Cu") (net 7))
 (via (at 96.8 69.5) (size 1.6) (drill 0.8) (layers "F.Cu" "B.Cu") (free yes) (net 1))
 (via (at 102.6 56.5) (size 1.6) (drill 0.8) (layers "F.Cu" "B.Cu") (free yes) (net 1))
 (via (at 98.3 54.3) (size 1.6) (drill 0.8) (layers "F.Cu" "B.Cu") (free yes) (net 1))
 (via (at 103.4 70.5) (size 1.6) (drill 0.8) (layers "F.Cu" "B.Cu") (free yes) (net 1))
 (via (at 116.2 69.8) (size 1.6) (drill 0.8) (layers "F.Cu" "B.Cu") (free yes) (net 1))
 (via (at 111.506 70.104) (size 1.6) (drill 0.8) (layers "F.Cu" "B.Cu") (free yes) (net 1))
 (via (at 116 56.5) (size 1.6) (drill 0.8) (layers "F.Cu" "B.Cu") (free yes) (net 1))
 (segment (start 101.445 58.674) (end 105.174 58.674) (width 0.3048) (layer "F.Cu") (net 5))
 (segment (start 105.174 58.674) (end 105.25 58.75) (width 0.3048) (layer "F.Cu") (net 5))
 (segment (start 107.702 71.969) (end 107.702 66.762) (width 0.3048) (layer "F.Cu") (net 2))
 (segment (start 107.67 66.73) (end 111.395 66.73) (width 0.3048) (layer "F.Cu") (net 2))
 (segment (start 107.702 66.762) (end 107.67 66.73) (width 0.3048) (layer "F.Cu") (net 2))
 (segment (start 111.506 67.564) (end 111.506 66.619) (width 0.3048) (layer "F.Cu") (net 2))
 (segment (start 111.395 66.73) (end 111.506 66.619) (width 0.3048) (layer "F.Cu") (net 2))
 (segment (start 111.506 64.77) (end 111.76 64.516) (width 0.3048) (layer "F.Cu") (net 4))
 (segment (start 111.506 65.659) (end 111.506 64.77) (width 0.3048) (layer "F.Cu") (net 4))
 (segment (start 111.76 62.941) (end 116.454107 62.941) (width 0.3048) (layer "F.Cu") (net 3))
 (segment (start 116.454107 62.941) (end 116.513107 63) (width 0.3048) (layer "F.Cu") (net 3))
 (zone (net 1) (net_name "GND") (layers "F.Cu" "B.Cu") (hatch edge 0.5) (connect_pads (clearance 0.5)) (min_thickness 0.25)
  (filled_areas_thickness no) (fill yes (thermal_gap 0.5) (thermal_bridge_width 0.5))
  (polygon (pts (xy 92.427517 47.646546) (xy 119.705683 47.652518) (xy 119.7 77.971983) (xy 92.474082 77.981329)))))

